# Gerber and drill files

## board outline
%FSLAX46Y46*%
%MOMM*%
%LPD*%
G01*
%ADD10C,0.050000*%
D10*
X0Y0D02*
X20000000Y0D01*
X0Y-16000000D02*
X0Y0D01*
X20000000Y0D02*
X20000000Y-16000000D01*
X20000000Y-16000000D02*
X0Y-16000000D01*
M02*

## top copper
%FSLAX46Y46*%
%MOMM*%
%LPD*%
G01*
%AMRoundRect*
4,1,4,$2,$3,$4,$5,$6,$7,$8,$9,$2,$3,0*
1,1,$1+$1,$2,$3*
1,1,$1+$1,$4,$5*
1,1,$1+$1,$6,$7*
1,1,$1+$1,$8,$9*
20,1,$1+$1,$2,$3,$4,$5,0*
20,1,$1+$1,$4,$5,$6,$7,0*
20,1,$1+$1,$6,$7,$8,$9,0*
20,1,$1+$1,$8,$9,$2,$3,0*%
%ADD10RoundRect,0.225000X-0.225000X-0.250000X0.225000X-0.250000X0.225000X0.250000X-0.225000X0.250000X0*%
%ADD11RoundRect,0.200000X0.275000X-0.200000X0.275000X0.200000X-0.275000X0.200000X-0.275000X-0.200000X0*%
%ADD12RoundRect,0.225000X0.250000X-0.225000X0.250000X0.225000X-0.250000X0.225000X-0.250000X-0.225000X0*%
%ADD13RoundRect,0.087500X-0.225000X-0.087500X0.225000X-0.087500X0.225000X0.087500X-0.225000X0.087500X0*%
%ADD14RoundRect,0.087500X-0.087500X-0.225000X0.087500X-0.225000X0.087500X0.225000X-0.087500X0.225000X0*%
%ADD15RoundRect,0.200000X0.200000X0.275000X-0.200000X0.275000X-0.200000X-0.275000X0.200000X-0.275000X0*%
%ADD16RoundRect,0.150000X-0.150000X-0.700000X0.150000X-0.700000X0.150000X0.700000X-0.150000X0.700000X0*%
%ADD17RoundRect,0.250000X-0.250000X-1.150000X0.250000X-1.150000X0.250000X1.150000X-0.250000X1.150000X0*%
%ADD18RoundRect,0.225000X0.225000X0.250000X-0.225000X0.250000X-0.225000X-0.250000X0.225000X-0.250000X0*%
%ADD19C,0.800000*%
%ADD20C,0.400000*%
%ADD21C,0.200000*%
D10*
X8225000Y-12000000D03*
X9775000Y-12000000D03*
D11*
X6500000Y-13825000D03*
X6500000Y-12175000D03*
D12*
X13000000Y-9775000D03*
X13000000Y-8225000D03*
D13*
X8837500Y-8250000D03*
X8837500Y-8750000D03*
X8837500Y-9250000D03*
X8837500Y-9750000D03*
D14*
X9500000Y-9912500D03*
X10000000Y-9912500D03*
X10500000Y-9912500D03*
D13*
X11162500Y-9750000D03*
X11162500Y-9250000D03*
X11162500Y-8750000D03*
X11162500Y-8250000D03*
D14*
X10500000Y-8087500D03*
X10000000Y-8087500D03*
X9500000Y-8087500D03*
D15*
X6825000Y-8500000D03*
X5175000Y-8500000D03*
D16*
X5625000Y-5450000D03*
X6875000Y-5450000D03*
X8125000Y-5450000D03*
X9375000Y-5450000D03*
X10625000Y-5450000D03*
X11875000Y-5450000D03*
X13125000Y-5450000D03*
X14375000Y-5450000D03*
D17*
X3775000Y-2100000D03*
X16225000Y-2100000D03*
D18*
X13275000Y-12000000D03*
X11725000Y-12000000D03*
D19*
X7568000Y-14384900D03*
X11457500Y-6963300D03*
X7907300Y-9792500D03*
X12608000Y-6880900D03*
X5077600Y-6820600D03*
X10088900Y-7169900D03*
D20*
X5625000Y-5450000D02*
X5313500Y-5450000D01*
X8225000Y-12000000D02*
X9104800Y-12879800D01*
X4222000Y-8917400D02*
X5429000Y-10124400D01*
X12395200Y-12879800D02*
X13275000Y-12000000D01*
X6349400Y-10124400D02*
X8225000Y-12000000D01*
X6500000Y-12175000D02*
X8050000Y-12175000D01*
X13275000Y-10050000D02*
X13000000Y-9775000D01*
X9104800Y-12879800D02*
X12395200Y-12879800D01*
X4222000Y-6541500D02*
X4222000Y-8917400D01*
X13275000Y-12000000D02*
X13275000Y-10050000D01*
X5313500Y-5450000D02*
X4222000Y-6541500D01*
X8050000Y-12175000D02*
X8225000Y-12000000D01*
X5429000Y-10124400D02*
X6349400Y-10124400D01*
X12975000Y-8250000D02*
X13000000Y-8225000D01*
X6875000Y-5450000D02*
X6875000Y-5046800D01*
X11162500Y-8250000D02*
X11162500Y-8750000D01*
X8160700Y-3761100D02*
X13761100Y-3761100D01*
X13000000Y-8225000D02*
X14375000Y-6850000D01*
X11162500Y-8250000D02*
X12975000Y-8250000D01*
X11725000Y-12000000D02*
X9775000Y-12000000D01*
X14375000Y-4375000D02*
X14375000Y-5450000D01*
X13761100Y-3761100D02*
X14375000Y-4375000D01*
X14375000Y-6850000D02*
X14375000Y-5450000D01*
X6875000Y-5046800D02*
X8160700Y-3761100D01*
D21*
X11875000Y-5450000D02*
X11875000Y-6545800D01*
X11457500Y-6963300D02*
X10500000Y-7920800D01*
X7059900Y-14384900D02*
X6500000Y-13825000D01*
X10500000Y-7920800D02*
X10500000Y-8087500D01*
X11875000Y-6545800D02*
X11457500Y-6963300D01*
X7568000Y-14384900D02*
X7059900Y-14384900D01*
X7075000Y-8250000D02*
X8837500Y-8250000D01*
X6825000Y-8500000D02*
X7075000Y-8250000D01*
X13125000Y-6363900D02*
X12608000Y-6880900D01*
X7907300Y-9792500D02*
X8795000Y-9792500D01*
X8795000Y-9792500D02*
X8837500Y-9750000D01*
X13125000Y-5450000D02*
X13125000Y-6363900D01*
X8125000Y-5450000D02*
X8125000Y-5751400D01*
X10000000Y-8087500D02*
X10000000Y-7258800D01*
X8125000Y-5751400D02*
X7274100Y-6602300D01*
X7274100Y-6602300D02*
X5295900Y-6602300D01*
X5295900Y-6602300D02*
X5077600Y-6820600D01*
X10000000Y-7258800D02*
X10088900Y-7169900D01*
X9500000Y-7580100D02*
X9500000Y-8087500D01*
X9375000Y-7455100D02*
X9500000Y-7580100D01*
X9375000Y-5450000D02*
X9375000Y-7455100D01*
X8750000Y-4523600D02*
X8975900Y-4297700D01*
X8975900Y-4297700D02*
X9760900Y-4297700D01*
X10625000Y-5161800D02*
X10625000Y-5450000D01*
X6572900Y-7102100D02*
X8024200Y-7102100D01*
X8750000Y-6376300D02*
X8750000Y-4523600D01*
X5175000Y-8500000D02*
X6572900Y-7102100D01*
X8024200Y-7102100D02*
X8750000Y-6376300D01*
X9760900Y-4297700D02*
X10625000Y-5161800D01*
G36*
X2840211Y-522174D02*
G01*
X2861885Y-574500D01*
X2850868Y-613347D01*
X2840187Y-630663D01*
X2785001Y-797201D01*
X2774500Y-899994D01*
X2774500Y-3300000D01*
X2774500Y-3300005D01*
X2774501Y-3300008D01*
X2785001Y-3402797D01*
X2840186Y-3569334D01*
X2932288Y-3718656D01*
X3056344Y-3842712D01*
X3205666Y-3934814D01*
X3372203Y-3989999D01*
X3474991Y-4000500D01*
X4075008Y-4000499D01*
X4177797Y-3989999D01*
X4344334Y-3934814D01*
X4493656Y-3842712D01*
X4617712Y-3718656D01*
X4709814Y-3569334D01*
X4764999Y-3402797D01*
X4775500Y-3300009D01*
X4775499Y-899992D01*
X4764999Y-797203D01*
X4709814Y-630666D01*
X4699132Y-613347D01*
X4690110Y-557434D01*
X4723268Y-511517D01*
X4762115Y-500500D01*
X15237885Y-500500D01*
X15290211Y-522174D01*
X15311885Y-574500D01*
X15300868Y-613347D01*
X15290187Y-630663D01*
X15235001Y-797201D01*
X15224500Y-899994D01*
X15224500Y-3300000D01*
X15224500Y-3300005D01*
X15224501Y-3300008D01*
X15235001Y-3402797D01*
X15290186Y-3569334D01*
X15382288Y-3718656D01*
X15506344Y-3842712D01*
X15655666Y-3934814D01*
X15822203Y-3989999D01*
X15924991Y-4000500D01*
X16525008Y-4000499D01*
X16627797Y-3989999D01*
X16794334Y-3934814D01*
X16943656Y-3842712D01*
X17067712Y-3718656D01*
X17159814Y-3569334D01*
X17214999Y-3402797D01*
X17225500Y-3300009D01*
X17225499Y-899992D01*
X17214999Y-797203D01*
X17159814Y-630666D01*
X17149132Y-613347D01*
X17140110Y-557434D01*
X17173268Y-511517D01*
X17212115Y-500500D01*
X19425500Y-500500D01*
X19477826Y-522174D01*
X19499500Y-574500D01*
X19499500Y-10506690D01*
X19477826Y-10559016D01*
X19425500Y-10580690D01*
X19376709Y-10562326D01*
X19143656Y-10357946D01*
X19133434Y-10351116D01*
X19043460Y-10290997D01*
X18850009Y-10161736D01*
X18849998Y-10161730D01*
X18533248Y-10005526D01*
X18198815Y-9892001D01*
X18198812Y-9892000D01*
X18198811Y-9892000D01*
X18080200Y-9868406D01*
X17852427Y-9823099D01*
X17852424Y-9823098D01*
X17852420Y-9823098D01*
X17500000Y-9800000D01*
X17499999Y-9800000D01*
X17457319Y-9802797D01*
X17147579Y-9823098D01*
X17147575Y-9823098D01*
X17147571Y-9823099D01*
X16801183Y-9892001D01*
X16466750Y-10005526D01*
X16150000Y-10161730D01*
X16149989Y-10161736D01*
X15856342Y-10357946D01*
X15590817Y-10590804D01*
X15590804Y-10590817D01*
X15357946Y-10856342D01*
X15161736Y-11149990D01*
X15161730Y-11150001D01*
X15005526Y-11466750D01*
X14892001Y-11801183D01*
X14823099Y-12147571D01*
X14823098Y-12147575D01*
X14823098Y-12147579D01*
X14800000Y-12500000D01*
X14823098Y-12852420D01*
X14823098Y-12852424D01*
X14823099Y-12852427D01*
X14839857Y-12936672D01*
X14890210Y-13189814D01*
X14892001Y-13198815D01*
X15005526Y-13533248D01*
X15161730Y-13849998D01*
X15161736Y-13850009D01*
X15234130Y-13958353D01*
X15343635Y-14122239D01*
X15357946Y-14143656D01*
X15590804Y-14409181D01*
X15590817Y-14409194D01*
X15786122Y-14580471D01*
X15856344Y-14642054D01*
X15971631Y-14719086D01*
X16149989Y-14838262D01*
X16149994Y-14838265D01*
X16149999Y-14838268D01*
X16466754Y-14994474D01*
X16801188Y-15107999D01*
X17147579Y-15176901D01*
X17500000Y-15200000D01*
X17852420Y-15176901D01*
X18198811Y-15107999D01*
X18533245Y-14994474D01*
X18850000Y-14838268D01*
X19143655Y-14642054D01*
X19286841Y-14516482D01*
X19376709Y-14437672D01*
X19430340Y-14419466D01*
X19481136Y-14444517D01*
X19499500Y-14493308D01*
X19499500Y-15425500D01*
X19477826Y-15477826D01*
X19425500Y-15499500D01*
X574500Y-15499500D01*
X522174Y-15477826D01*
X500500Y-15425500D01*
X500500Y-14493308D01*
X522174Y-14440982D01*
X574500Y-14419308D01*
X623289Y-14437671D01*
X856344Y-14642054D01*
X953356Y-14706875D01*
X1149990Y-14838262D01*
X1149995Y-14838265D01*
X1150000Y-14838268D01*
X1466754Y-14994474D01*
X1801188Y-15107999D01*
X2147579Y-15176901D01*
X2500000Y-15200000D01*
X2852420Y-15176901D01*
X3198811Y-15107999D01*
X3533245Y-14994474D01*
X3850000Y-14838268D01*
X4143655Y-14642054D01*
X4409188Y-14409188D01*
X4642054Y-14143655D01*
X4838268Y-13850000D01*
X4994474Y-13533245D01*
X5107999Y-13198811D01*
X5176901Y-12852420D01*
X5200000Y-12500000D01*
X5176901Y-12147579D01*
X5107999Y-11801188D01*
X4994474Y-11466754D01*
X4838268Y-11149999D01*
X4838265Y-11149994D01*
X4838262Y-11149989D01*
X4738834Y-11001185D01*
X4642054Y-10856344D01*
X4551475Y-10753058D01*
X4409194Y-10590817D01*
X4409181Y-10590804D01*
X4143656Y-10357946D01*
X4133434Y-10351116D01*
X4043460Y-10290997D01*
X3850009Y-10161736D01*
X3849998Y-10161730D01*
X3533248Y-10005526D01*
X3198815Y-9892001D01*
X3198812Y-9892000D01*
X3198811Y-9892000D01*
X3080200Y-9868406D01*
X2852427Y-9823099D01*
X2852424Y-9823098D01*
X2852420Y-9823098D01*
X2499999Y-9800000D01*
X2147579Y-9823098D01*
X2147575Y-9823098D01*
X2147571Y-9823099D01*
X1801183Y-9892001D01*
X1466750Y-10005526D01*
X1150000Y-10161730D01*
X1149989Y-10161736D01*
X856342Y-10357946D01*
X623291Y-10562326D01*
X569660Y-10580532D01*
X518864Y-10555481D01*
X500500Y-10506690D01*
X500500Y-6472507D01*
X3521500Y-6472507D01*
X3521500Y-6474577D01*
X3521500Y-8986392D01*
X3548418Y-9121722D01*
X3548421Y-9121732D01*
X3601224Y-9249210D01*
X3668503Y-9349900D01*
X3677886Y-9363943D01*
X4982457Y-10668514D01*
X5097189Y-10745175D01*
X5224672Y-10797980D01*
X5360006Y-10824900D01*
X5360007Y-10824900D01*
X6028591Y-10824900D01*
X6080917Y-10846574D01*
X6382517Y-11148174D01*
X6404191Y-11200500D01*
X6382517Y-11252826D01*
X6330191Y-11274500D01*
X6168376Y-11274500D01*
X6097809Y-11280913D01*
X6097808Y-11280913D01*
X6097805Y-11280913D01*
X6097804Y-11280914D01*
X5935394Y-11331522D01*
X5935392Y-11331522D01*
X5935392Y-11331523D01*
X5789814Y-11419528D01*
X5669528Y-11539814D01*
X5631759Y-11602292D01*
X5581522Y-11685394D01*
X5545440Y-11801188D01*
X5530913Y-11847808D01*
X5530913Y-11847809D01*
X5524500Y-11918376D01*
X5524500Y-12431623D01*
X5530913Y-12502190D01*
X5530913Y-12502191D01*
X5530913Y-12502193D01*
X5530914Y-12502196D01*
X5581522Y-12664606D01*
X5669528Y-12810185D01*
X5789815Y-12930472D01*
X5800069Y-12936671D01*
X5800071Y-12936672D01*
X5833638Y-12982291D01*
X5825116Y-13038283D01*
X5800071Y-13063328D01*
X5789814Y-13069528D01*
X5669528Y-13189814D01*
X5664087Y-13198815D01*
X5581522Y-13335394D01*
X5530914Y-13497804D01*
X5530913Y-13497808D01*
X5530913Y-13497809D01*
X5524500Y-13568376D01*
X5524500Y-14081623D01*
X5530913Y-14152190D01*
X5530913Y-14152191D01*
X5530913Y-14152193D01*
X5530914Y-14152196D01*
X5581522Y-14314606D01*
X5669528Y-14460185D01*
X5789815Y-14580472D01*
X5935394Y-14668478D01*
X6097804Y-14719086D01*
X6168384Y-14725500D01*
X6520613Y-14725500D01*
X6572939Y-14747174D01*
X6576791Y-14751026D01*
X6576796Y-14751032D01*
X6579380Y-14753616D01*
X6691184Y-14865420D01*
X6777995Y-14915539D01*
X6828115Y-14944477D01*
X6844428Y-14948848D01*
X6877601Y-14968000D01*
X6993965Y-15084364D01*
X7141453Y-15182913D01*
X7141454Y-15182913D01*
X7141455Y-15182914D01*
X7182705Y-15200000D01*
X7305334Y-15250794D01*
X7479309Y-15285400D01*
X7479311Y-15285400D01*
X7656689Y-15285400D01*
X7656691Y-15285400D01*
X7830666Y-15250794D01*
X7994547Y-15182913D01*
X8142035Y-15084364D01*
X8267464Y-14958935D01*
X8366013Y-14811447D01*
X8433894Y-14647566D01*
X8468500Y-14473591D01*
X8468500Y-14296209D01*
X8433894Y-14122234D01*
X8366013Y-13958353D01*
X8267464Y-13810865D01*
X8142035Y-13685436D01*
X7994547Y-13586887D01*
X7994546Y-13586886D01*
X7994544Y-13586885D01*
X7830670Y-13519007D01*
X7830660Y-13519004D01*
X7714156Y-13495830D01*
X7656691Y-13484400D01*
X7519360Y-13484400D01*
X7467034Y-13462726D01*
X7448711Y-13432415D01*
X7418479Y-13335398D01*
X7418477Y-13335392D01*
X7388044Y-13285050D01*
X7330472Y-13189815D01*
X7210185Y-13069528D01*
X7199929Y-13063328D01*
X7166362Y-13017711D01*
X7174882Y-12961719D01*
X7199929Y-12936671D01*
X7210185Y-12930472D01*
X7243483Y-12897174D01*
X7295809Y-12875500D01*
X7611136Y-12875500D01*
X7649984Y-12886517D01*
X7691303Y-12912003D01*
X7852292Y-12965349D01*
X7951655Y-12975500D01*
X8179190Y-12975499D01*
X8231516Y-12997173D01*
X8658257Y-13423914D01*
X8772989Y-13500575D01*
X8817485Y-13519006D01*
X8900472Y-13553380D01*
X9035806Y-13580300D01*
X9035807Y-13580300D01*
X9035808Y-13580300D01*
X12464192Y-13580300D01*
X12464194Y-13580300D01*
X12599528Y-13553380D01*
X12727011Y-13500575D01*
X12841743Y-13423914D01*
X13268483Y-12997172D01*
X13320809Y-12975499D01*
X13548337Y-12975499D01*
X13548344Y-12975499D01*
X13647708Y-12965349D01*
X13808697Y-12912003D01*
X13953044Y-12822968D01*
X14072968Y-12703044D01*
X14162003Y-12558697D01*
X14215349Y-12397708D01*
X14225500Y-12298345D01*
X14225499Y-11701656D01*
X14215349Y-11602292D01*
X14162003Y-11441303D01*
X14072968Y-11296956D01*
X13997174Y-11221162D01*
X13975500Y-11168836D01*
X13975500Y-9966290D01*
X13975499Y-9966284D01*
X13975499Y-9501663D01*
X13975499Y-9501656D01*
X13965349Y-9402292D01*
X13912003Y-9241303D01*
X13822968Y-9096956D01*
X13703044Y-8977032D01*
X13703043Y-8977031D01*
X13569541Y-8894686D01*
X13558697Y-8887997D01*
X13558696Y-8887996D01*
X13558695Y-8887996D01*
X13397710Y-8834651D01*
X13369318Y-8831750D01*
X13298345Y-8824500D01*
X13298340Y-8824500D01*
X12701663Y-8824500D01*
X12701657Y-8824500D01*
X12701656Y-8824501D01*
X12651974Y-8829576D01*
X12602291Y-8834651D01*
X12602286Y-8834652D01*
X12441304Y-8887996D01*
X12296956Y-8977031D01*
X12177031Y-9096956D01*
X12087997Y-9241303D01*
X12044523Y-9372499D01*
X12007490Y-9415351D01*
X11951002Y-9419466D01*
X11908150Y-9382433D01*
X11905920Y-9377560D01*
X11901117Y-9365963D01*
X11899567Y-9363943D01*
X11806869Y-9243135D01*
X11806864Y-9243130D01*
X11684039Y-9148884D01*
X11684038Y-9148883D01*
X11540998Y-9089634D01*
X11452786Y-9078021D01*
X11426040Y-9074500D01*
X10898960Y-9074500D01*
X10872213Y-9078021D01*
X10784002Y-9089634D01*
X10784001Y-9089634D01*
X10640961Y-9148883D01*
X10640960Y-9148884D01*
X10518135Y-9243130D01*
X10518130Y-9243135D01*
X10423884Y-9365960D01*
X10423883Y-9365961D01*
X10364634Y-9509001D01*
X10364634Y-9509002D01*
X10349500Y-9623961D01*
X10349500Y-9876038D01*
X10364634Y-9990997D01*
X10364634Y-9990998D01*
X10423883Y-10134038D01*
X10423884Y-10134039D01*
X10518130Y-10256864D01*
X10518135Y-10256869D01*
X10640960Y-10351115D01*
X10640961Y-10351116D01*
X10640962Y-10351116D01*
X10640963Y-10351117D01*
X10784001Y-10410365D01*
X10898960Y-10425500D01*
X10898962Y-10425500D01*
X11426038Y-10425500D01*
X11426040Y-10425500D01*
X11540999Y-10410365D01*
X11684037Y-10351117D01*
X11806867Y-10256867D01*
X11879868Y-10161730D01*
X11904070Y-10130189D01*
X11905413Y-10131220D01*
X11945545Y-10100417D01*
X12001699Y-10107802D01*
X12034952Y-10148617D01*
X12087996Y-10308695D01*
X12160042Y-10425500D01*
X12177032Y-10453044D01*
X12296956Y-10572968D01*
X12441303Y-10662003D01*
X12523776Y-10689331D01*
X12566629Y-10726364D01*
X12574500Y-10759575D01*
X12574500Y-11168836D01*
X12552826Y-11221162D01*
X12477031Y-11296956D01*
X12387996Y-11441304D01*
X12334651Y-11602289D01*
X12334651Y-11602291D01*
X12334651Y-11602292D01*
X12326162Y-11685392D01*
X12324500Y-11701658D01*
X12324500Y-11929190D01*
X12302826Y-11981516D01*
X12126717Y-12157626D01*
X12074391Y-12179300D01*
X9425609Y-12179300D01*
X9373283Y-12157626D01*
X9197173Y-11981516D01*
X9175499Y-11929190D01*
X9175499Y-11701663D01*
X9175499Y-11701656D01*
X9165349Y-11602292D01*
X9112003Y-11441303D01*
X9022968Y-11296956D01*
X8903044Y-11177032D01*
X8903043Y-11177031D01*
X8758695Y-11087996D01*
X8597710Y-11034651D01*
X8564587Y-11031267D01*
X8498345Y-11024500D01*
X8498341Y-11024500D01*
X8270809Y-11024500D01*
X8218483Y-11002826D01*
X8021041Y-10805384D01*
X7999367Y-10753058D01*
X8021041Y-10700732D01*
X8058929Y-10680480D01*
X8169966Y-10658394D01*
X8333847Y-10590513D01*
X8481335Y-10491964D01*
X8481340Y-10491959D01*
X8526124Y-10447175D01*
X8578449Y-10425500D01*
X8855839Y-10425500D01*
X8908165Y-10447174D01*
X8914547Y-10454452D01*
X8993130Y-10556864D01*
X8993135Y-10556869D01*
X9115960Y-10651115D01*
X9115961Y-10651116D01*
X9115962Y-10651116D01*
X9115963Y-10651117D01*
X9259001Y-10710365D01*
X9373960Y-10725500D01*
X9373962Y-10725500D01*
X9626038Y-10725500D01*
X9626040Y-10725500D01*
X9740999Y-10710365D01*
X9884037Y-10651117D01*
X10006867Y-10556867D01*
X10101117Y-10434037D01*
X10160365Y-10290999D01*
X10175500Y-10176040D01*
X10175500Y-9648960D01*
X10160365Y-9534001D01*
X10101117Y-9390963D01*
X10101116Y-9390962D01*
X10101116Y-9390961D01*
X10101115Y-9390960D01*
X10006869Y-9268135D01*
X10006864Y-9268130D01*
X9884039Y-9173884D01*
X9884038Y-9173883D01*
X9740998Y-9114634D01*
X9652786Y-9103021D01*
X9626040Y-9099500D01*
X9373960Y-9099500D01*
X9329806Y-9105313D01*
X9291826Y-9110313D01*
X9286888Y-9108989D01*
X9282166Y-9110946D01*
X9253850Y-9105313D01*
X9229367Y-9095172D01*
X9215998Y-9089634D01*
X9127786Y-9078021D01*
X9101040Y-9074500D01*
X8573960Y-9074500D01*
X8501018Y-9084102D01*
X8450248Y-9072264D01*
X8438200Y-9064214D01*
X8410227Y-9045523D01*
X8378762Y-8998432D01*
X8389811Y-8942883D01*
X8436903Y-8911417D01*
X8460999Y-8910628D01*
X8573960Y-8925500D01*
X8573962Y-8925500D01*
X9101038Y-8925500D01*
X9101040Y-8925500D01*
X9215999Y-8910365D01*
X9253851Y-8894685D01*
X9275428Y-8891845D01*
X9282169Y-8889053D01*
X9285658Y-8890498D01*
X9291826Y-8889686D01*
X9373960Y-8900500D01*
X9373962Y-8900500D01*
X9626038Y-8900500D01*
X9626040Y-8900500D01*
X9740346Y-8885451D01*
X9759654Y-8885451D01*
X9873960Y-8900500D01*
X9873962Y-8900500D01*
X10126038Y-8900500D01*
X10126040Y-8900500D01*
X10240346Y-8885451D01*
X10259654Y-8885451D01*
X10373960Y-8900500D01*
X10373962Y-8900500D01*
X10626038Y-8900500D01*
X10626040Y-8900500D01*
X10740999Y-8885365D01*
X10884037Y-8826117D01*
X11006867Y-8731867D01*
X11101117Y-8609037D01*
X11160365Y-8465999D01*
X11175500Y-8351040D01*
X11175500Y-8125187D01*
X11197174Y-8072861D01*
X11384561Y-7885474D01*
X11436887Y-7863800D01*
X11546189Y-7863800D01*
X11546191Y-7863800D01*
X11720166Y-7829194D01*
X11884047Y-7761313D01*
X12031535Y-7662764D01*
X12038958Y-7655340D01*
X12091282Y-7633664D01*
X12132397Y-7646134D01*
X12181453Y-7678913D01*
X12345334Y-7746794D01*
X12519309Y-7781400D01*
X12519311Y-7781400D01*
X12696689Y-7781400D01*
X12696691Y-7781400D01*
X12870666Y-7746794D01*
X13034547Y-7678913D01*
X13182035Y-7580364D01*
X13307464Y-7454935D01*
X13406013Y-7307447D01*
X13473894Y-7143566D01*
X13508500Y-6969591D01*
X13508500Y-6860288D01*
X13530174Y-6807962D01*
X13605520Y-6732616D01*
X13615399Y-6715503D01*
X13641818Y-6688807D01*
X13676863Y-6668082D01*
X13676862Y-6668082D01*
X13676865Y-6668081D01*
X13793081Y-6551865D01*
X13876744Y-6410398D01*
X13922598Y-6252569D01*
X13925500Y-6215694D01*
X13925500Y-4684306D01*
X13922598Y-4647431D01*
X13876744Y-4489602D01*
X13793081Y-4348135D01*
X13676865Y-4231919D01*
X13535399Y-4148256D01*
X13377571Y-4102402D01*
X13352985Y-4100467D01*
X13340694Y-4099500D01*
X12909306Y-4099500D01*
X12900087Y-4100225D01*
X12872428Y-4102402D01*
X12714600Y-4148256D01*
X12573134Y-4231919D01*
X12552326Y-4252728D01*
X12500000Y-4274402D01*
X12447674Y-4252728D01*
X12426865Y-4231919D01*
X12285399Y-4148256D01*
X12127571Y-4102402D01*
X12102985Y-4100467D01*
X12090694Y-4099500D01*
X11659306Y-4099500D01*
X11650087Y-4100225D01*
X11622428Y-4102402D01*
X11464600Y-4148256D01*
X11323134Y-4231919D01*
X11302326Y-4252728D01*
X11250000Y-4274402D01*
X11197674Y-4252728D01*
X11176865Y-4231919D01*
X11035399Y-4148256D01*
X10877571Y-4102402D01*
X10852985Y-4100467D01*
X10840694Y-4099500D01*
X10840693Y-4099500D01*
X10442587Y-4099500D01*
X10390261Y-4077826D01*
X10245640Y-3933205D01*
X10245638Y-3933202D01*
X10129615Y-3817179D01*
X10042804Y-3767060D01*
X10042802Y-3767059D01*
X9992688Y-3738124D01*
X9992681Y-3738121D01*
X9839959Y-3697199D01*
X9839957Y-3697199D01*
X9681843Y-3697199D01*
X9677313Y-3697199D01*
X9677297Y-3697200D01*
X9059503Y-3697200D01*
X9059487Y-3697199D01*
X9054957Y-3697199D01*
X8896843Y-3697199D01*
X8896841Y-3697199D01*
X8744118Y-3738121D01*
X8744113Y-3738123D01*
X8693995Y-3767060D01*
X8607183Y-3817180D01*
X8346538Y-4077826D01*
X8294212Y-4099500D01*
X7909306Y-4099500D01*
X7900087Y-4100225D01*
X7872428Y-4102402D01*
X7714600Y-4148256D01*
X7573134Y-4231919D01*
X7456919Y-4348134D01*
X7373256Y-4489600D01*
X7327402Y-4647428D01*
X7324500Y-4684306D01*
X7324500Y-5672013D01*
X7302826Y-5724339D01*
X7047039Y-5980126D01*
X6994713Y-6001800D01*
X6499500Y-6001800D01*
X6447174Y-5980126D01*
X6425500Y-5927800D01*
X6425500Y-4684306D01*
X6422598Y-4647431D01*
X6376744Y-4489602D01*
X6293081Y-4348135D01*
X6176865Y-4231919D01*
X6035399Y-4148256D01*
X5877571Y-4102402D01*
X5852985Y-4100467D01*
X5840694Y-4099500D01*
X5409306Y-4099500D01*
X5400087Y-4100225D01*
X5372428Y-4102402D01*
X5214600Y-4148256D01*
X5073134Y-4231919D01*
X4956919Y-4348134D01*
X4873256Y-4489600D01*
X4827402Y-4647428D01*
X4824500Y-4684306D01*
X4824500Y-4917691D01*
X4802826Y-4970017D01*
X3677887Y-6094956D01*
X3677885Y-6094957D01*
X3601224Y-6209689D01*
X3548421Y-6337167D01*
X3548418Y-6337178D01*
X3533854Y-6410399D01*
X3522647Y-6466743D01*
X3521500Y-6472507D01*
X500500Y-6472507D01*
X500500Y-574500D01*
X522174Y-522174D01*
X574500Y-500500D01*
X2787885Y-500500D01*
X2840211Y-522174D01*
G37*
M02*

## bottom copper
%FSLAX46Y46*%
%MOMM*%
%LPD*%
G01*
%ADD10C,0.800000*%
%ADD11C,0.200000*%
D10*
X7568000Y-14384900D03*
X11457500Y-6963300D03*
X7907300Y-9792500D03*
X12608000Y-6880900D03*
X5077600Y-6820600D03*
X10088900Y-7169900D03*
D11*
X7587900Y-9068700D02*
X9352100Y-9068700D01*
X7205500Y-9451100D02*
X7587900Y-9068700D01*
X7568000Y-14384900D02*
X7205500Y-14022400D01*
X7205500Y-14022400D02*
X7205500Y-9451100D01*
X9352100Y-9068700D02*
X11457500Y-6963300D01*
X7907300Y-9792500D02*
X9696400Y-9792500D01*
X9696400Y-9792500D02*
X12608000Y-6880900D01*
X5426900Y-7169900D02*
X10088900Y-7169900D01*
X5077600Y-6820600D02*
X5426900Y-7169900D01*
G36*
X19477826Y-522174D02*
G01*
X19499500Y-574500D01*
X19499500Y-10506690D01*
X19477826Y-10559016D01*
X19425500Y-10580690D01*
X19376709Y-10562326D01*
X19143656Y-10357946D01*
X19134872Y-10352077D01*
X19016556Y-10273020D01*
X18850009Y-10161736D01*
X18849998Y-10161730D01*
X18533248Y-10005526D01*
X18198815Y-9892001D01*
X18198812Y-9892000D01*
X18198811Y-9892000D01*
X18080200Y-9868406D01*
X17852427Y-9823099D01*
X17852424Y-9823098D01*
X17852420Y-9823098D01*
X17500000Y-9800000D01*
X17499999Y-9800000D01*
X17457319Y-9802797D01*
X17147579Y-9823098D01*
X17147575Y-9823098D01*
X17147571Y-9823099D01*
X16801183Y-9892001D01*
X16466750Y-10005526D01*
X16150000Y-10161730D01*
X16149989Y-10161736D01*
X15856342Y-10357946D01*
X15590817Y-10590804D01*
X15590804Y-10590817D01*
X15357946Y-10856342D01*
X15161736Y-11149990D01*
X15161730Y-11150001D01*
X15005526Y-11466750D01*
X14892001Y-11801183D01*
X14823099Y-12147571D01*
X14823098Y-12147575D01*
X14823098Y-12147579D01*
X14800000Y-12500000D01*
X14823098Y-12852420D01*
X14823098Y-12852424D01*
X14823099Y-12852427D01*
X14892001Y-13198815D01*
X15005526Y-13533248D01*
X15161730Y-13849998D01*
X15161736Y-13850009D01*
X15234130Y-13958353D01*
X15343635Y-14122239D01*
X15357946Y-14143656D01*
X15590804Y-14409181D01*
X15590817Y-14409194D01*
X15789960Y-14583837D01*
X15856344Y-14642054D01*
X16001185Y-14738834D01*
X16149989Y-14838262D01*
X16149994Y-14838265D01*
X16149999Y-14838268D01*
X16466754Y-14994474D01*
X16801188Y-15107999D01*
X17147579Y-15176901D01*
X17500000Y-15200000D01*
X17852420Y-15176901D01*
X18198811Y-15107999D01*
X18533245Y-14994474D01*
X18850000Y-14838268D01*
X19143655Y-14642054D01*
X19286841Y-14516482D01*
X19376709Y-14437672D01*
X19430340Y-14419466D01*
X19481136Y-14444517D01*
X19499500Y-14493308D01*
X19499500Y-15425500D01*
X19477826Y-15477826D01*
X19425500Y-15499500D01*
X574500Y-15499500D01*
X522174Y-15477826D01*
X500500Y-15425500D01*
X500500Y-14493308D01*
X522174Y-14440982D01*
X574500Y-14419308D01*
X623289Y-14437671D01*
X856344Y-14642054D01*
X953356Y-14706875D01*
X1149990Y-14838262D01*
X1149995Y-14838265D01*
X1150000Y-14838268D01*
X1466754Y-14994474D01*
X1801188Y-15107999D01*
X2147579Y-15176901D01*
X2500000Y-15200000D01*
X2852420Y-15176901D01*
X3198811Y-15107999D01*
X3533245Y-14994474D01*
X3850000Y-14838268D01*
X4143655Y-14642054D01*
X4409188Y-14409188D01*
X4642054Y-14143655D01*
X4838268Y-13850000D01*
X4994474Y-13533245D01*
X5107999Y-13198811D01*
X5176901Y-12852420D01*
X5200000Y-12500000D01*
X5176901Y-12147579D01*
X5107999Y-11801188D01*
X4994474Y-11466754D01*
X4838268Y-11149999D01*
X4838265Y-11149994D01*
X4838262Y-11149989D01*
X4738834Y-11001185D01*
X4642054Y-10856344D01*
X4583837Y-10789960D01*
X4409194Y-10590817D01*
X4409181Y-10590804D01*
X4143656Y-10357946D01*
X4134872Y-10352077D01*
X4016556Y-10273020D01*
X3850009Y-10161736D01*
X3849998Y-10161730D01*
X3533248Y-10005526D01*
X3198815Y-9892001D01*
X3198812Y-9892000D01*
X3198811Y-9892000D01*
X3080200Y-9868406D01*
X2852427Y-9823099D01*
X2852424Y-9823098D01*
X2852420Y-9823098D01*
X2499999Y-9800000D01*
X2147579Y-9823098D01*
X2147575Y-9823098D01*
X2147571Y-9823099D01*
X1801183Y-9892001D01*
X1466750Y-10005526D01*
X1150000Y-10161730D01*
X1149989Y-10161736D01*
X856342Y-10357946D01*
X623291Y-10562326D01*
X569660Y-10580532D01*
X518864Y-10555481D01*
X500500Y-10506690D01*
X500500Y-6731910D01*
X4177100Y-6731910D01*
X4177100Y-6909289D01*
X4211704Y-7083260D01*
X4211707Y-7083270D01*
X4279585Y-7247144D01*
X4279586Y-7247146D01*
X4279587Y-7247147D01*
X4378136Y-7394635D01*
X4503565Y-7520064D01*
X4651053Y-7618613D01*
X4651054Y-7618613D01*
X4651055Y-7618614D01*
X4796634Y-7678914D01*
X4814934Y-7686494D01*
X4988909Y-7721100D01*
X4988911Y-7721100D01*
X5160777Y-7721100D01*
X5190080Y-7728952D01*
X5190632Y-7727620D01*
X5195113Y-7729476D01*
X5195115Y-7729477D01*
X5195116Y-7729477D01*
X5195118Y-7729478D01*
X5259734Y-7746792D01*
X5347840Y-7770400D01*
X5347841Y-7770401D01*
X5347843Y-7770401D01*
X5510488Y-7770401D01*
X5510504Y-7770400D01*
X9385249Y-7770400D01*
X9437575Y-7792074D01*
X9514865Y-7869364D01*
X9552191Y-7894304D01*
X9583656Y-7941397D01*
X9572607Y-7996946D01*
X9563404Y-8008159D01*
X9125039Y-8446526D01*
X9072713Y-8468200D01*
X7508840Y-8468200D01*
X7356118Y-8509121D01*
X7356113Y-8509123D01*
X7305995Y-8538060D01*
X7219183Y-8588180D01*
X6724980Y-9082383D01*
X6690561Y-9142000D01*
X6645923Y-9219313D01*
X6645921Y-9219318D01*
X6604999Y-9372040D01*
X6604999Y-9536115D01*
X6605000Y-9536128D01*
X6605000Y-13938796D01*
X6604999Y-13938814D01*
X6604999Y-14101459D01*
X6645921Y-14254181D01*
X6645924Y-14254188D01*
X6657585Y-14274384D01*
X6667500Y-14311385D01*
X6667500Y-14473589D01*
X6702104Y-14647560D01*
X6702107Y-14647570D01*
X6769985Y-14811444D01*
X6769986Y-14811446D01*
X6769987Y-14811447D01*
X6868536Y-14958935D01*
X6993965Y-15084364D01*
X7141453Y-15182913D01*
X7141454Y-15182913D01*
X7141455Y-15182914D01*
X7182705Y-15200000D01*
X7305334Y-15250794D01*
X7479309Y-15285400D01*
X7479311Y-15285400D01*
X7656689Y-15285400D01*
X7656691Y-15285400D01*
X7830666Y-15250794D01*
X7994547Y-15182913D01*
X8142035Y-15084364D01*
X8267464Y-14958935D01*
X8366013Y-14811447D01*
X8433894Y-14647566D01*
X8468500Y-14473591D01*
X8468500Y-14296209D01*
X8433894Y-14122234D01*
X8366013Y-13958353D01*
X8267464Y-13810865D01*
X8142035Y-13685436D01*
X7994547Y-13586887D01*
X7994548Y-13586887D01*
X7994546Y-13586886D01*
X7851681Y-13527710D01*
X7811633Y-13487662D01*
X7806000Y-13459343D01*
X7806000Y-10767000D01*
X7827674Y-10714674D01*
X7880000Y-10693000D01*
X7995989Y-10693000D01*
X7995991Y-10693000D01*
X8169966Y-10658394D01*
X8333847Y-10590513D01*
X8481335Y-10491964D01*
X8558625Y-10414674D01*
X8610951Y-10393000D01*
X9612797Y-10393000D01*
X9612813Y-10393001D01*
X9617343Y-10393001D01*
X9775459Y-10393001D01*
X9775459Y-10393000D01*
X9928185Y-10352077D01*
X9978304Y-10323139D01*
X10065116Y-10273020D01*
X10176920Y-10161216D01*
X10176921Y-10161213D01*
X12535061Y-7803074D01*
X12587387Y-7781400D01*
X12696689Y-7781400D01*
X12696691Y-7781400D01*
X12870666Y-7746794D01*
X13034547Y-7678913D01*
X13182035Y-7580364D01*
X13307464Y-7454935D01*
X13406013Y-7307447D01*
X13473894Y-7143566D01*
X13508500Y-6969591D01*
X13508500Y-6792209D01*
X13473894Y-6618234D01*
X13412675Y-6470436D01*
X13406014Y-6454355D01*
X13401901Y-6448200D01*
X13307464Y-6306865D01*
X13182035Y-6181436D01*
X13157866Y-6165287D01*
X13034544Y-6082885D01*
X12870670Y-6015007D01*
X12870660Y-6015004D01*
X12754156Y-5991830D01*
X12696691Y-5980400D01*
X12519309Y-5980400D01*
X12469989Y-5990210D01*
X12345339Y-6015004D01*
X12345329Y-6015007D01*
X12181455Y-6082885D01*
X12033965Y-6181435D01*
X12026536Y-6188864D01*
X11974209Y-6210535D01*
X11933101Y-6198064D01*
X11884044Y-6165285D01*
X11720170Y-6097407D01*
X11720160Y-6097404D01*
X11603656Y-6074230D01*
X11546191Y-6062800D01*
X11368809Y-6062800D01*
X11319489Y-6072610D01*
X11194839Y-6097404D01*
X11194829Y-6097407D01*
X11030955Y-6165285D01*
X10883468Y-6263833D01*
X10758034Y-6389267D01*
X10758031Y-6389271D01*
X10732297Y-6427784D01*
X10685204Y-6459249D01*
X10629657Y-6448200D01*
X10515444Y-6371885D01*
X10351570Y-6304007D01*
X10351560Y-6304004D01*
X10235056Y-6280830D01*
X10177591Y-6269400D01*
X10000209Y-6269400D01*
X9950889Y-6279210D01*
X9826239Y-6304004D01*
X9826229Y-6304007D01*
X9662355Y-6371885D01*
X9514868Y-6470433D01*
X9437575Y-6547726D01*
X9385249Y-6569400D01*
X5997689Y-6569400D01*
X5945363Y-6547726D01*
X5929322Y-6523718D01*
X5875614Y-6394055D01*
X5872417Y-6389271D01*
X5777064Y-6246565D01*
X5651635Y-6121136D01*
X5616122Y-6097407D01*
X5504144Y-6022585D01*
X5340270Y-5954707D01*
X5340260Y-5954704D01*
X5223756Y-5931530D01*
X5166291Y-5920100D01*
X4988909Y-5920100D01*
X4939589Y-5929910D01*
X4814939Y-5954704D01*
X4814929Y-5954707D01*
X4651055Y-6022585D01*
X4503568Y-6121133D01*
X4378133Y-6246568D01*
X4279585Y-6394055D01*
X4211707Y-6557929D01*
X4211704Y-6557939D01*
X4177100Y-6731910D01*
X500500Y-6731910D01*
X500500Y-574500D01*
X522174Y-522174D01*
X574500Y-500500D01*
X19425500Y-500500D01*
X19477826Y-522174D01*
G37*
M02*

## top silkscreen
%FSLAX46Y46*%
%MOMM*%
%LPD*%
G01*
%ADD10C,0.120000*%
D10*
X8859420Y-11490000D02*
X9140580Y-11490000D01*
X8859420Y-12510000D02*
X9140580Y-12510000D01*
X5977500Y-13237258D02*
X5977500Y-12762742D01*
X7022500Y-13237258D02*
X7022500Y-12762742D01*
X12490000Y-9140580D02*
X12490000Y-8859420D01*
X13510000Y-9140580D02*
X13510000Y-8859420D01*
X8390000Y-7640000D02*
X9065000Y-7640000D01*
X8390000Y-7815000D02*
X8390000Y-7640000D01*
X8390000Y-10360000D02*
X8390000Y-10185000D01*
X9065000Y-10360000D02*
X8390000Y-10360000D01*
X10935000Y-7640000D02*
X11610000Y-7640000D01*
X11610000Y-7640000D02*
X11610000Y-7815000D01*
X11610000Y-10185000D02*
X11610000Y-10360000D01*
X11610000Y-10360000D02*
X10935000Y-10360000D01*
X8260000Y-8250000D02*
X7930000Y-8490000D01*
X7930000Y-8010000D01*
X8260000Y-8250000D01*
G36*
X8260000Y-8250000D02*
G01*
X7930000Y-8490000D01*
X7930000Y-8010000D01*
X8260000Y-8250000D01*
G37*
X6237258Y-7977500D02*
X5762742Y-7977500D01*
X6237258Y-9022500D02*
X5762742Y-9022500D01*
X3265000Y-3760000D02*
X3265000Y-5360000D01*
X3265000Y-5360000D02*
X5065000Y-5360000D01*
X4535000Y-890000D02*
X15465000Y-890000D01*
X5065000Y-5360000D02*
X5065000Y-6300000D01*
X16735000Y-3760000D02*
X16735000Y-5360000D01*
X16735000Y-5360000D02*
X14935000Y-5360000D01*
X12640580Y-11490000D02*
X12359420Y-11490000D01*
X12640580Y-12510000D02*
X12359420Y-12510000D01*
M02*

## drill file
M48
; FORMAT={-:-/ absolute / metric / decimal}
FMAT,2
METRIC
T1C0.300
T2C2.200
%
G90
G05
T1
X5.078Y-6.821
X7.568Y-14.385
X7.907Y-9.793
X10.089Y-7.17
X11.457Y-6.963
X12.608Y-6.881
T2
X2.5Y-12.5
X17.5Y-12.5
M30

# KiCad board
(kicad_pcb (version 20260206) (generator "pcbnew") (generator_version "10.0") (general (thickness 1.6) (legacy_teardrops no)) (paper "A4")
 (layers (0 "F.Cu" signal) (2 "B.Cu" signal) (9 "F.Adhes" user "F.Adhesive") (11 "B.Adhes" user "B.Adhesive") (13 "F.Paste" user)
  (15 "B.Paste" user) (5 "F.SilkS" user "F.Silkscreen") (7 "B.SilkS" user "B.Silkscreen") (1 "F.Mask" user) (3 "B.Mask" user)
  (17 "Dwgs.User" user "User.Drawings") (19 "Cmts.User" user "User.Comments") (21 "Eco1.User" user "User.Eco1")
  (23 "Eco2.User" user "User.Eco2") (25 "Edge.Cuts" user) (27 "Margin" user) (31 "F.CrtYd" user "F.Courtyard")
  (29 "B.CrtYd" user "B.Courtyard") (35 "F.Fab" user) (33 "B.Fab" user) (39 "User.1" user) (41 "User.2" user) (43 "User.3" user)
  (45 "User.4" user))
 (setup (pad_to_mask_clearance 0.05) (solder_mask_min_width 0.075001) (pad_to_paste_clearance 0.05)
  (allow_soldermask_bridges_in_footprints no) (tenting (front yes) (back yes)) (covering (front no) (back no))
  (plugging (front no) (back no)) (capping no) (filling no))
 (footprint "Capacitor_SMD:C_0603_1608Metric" (layer "F.Cu") (at 9 12)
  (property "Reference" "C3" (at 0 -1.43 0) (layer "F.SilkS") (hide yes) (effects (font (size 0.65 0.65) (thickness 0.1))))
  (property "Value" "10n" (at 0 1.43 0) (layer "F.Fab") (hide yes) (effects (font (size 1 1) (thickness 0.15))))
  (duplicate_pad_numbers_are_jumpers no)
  (fp_line (start -0.14058 -0.51) (end 0.14058 -0.51) (stroke (width 0.12) (type solid)) (layer "F.SilkS"))
  (fp_line (start -0.14058 0.51) (end 0.14058 0.51) (stroke (width 0.12) (type solid)) (layer "F.SilkS"))
  (pad "1" smd roundrect (at -0.775 0) (size 0.9 0.95) (layers "F.Cu" "F.Mask" "F.Paste") (roundrect_rratio 0.25) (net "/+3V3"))
  (pad "2" smd roundrect (at 0.775 0) (size 0.9 0.95) (layers "F.Cu" "F.Mask" "F.Paste") (roundrect_rratio 0.25) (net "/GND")
   (zone_connect 2)))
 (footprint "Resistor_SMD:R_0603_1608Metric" (layer "F.Cu") (at 6.5 13 90)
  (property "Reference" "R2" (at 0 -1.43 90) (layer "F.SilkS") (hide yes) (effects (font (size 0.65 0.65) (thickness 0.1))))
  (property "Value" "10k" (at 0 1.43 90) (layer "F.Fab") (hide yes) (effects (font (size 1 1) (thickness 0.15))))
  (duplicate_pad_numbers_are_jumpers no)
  (fp_line (start -0.237258 -0.5225) (end 0.237258 -0.5225) (stroke (width 0.12) (type solid)) (layer "F.SilkS"))
  (fp_line (start -0.237258 0.5225) (end 0.237258 0.5225) (stroke (width 0.12) (type solid)) (layer "F.SilkS"))
  (pad "1" smd roundrect (at -0.825 0 90) (size 0.8 0.95) (layers "F.Cu" "F.Mask" "F.Paste") (roundrect_rratio 0.25) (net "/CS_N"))
  (pad "2" smd roundrect (at 0.825 0 90) (size 0.8 0.95) (layers "F.Cu" "F.Mask" "F.Paste") (roundrect_rratio 0.25) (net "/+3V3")))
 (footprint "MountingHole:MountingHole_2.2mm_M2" (layer "F.Cu") (at 2.5 12.5)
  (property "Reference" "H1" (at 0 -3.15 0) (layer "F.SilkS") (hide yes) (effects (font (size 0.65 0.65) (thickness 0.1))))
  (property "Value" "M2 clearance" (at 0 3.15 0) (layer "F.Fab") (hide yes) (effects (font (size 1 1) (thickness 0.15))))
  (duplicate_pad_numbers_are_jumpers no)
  (pad "" np_thru_hole circle (at 0 0) (size 2.2 2.2) (drill 2.2) (layers "*.Cu" "*.Mask")))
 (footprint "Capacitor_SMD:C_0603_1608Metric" (layer "F.Cu") (at 13 9 90)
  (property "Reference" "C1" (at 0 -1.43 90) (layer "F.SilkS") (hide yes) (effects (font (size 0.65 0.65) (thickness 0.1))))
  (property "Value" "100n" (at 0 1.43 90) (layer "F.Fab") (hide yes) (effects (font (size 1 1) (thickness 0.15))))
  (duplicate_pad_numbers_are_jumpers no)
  (fp_line (start -0.14058 -0.51) (end 0.14058 -0.51) (stroke (width 0.12) (type solid)) (layer "F.SilkS"))
  (fp_line (start -0.14058 0.51) (end 0.14058 0.51) (stroke (width 0.12) (type solid)) (layer "F.SilkS"))
  (pad "1" smd roundrect (at -0.775 0 90) (size 0.9 0.95) (layers "F.Cu" "F.Mask" "F.Paste") (roundrect_rratio 0.25) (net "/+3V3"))
  (pad "2" smd roundrect (at 0.775 0 90) (size 0.9 0.95) (layers "F.Cu" "F.Mask" "F.Paste") (roundrect_rratio 0.25) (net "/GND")
   (zone_connect 2)))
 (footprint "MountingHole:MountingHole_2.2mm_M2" (layer "F.Cu") (at 17.5 12.5)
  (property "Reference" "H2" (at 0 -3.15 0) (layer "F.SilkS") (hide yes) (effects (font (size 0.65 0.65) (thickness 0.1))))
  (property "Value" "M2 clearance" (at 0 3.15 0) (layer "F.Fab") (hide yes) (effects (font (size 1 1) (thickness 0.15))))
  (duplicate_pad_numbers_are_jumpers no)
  (pad "" np_thru_hole circle (at 0 0) (size 2.2 2.2) (drill 2.2) (layers "*.Cu" "*.Mask")))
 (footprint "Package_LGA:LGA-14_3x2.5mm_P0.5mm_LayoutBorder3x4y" (layer "F.Cu") (at 10 9)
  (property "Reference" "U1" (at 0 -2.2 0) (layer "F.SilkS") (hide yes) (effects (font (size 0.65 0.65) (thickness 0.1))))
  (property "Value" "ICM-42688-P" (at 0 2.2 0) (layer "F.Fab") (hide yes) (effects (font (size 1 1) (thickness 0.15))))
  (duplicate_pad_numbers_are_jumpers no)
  (fp_line (start -1.61 -1.36) (end -0.935 -1.36) (stroke (width 0.12) (type solid)) (layer "F.SilkS"))
  (fp_line (start -1.61 -1.185) (end -1.61 -1.36) (stroke (width 0.12) (type solid)) (layer "F.SilkS"))
  (fp_line (start -1.61 1.36) (end -1.61 1.185) (stroke (width 0.12) (type solid)) (layer "F.SilkS"))
  (fp_line (start -0.935 1.36) (end -1.61 1.36) (stroke (width 0.12) (type solid)) (layer "F.SilkS"))
  (fp_line (start 0.935 -1.36) (end 1.61 -1.36) (stroke (width 0.12) (type solid)) (layer "F.SilkS"))
  (fp_line (start 1.61 -1.36) (end 1.61 -1.185) (stroke (width 0.12) (type solid)) (layer "F.SilkS"))
  (fp_line (start 1.61 1.185) (end 1.61 1.36) (stroke (width 0.12) (type solid)) (layer "F.SilkS"))
  (fp_line (start 1.61 1.36) (end 0.935 1.36) (stroke (width 0.12) (type solid)) (layer "F.SilkS"))
  (fp_poly (pts (xy -1.74 -0.75) (xy -2.07 -0.51) (xy -2.07 -0.99)) (stroke (width 0.12) (type solid)) (fill yes) (layer "F.SilkS"))
  (pad "1" smd roundrect (at -1.1625 -0.75) (size 0.625 0.35) (layers "F.Cu" "F.Mask" "F.Paste") (roundrect_rratio 0.25) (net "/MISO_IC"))
  (pad "2" smd roundrect (at -1.1625 -0.25) (size 0.625 0.35) (layers "F.Cu" "F.Mask" "F.Paste") (roundrect_rratio 0.25) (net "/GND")
   (zone_connect 2))
  (pad "3" smd roundrect (at -1.1625 0.25) (size 0.625 0.35) (layers "F.Cu" "F.Mask" "F.Paste") (roundrect_rratio 0.25) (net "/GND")
   (zone_connect 2))
  (pad "4" smd roundrect (at -1.1625 0.75) (size 0.625 0.35) (layers "F.Cu" "F.Mask" "F.Paste") (roundrect_rratio 0.25) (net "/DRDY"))
  (pad "5" smd roundrect (at -0.5 0.9125) (size 0.35 0.625) (layers "F.Cu" "F.Mask" "F.Paste") (roundrect_rratio 0.25) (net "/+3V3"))
  (pad "6" smd roundrect (at 0 0.9125) (size 0.35 0.625) (layers "F.Cu" "F.Mask" "F.Paste") (roundrect_rratio 0.25) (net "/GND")
   (zone_connect 2))
  (pad "7" smd roundrect (at 0.5 0.9125) (size 0.35 0.625) (layers "F.Cu" "F.Mask" "F.Paste") (roundrect_rratio 0.25) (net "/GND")
   (zone_connect 2))
  (pad "8" smd roundrect (at 1.1625 0.75) (size 0.625 0.35) (layers "F.Cu" "F.Mask" "F.Paste") (roundrect_rratio 0.25) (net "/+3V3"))
  (pad "9" smd roundrect (at 1.1625 0.25) (size 0.625 0.35) (layers "F.Cu" "F.Mask" "F.Paste") (roundrect_rratio 0.25) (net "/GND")
   (zone_connect 2))
  (pad "10" smd roundrect (at 1.1625 -0.25) (size 0.625 0.35) (layers "F.Cu" "F.Mask" "F.Paste") (roundrect_rratio 0.25) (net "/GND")
   (zone_connect 2))
  (pad "11" smd roundrect (at 1.1625 -0.75) (size 0.625 0.35) (layers "F.Cu" "F.Mask" "F.Paste") (roundrect_rratio 0.25) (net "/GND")
   (zone_connect 2))
  (pad "12" smd roundrect (at 0.5 -0.9125) (size 0.35 0.625) (layers "F.Cu" "F.Mask" "F.Paste") (roundrect_rratio 0.25) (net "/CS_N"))
  (pad "13" smd roundrect (at 0 -0.9125) (size 0.35 0.625) (layers "F.Cu" "F.Mask" "F.Paste") (roundrect_rratio 0.25) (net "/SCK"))
  (pad "14" smd roundrect (at -0.5 -0.9125) (size 0.35 0.625) (layers "F.Cu" "F.Mask" "F.Paste") (roundrect_rratio 0.25) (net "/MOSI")))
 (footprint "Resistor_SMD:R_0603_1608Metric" (layer "F.Cu") (at 6 8.5 180)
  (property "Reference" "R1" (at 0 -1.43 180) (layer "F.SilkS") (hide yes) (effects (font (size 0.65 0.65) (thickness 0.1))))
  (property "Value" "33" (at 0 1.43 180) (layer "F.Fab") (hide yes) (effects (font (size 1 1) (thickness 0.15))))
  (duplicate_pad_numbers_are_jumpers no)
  (fp_line (start -0.237258 0.5225) (end 0.237258 0.5225) (stroke (width 0.12) (type solid)) (layer "F.SilkS"))
  (fp_line (start -0.237258 -0.5225) (end 0.237258 -0.5225) (stroke (width 0.12) (type solid)) (layer "F.SilkS"))
  (pad "1" smd roundrect (at -0.825 0 180) (size 0.8 0.95) (layers "F.Cu" "F.Mask" "F.Paste") (roundrect_rratio 0.25) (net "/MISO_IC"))
  (pad "2" smd roundrect (at 0.825 0 180) (size 0.8 0.95) (layers "F.Cu" "F.Mask" "F.Paste") (roundrect_rratio 0.25) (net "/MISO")))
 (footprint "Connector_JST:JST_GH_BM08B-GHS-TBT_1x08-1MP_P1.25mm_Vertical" (layer "F.Cu") (at 10 3.5)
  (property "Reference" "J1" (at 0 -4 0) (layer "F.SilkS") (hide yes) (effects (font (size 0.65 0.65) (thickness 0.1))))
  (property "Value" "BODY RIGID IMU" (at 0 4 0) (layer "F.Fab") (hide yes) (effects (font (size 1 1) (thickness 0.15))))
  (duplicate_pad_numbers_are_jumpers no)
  (fp_line (start -6.735 0.26) (end -6.735 1.86) (stroke (width 0.12) (type solid)) (layer "F.SilkS"))
  (fp_line (start -6.735 1.86) (end -4.935 1.86) (stroke (width 0.12) (type solid)) (layer "F.SilkS"))
  (fp_line (start -5.465 -2.61) (end 5.465 -2.61) (stroke (width 0.12) (type solid)) (layer "F.SilkS"))
  (fp_line (start -4.935 1.86) (end -4.935 2.8) (stroke (width 0.12) (type solid)) (layer "F.SilkS"))
  (fp_line (start 6.735 0.26) (end 6.735 1.86) (stroke (width 0.12) (type solid)) (layer "F.SilkS"))
  (fp_line (start 6.735 1.86) (end 4.935 1.86) (stroke (width 0.12) (type solid)) (layer "F.SilkS"))
  (pad "1" smd roundrect (at -4.375 1.95) (size 0.6 1.7) (layers "F.Cu" "F.Mask" "F.Paste") (roundrect_rratio 0.25) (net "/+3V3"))
  (pad "2" smd roundrect (at -3.125 1.95) (size 0.6 1.7) (layers "F.Cu" "F.Mask" "F.Paste") (roundrect_rratio 0.25) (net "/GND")
   (zone_connect 2))
  (pad "3" smd roundrect (at -1.875 1.95) (size 0.6 1.7) (layers "F.Cu" "F.Mask" "F.Paste") (roundrect_rratio 0.25) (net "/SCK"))
  (pad "4" smd roundrect (at -0.625 1.95) (size 0.6 1.7) (layers "F.Cu" "F.Mask" "F.Paste") (roundrect_rratio 0.25) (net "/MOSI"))
  (pad "5" smd roundrect (at 0.625 1.95) (size 0.6 1.7) (layers "F.Cu" "F.Mask" "F.Paste") (roundrect_rratio 0.25) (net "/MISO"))
  (pad "6" smd roundrect (at 1.875 1.95) (size 0.6 1.7) (layers "F.Cu" "F.Mask" "F.Paste") (roundrect_rratio 0.25) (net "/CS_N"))
  (pad "7" smd roundrect (at 3.125 1.95) (size 0.6 1.7) (layers "F.Cu" "F.Mask" "F.Paste") (roundrect_rratio 0.25) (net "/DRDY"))
  (pad "8" smd roundrect (at 4.375 1.95) (size 0.6 1.7) (layers "F.Cu" "F.Mask" "F.Paste") (roundrect_rratio 0.25) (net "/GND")
   (zone_connect 2))
  (pad "MP" smd roundrect (at -6.225 -1.4) (size 1 2.8) (layers "F.Cu" "F.Mask" "F.Paste") (roundrect_rratio 0.25))
  (pad "MP" smd roundrect (at 6.225 -1.4) (size 1 2.8) (layers "F.Cu" "F.Mask" "F.Paste") (roundrect_rratio 0.25)))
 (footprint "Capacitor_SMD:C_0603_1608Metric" (layer "F.Cu") (at 12.5 12 180)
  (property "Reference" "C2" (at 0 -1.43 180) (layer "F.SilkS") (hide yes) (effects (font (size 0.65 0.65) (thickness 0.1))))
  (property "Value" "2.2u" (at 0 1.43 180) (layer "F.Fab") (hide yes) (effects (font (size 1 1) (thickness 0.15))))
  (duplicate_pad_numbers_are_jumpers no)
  (fp_line (start -0.14058 0.51) (end 0.14058 0.51) (stroke (width 0.12) (type solid)) (layer "F.SilkS"))
  (fp_line (start -0.14058 -0.51) (end 0.14058 -0.51) (stroke (width 0.12) (type solid)) (layer "F.SilkS"))
  (pad "1" smd roundrect (at -0.775 0 180) (size 0.9 0.95) (layers "F.Cu" "F.Mask" "F.Paste") (roundrect_rratio 0.25) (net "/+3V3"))
  (pad "2" smd roundrect (at 0.775 0 180) (size 0.9 0.95) (layers "F.Cu" "F.Mask" "F.Paste") (roundrect_rratio 0.25) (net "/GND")
   (zone_connect 2)))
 (gr_line (start 0 0) (end 20 0) (stroke (width 0.05) (type default)) (layer "Edge.Cuts"))
 (gr_line (start 0 16) (end 0 0) (stroke (width 0.05) (type default)) (layer "Edge.Cuts"))
 (gr_line (start 20 0) (end 20 16) (stroke (width 0.05) (type default)) (layer "Edge.Cuts"))
 (gr_line (start 20 16) (end 0 16) (stroke (width 0.05) (type default)) (layer "Edge.Cuts"))
 (segment (start 5.625 5.45) (end 5.3135 5.45) (width 0.4) (layer "F.Cu") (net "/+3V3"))
 (segment (start 8.225 12) (end 9.1048 12.8798) (width 0.4) (layer "F.Cu") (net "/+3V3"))
 (segment (start 4.222 8.9174) (end 5.429 10.1244) (width 0.4) (layer "F.Cu") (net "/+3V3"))
 (segment (start 12.3952 12.8798) (end 13.275 12) (width 0.4) (layer "F.Cu") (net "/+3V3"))
 (segment (start 6.3494 10.1244) (end 8.225 12) (width 0.4) (layer "F.Cu") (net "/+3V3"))
 (segment (start 6.5 12.175) (end 8.05 12.175) (width 0.4) (layer "F.Cu") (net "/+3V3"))
 (segment (start 13.275 10.05) (end 13 9.775) (width 0.4) (layer "F.Cu") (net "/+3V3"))
 (segment (start 9.1048 12.8798) (end 12.3952 12.8798) (width 0.4) (layer "F.Cu") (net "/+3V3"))
 (segment (start 4.222 6.5415) (end 4.222 8.9174) (width 0.4) (layer "F.Cu") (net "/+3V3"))
 (segment (start 13.275 12) (end 13.275 10.05) (width 0.4) (layer "F.Cu") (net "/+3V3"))
 (segment (start 5.3135 5.45) (end 4.222 6.5415) (width 0.4) (layer "F.Cu") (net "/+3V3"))
 (segment (start 8.05 12.175) (end 8.225 12) (width 0.4) (layer "F.Cu") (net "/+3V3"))
 (segment (start 5.429 10.1244) (end 6.3494 10.1244) (width 0.4) (layer "F.Cu") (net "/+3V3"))
 (segment (start 12.975 8.25) (end 13 8.225) (width 0.4) (layer "F.Cu") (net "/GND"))
 (segment (start 6.875 5.45) (end 6.875 5.0468) (width 0.4) (layer "F.Cu") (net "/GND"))
 (segment (start 11.1625 8.25) (end 11.1625 8.75) (width 0.4) (layer "F.Cu") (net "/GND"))
 (segment (start 8.1607 3.7611) (end 13.7611 3.7611) (width 0.4) (layer "F.Cu") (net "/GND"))
 (segment (start 13 8.225) (end 14.375 6.85) (width 0.4) (layer "F.Cu") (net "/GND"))
 (segment (start 11.1625 8.25) (end 12.975 8.25) (width 0.4) (layer "F.Cu") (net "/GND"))
 (segment (start 11.725 12) (end 9.775 12) (width 0.4) (layer "F.Cu") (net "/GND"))
 (segment (start 14.375 4.375) (end 14.375 5.45) (width 0.4) (layer "F.Cu") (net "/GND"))
 (segment (start 13.7611 3.7611) (end 14.375 4.375) (width 0.4) (layer "F.Cu") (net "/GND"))
 (segment (start 14.375 6.85) (end 14.375 5.45) (width 0.4) (layer "F.Cu") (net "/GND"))
 (segment (start 6.875 5.0468) (end 8.1607 3.7611) (width 0.4) (layer "F.Cu") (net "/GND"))
 (segment (start 11.875 5.45) (end 11.875 6.5458) (width 0.2) (layer "F.Cu") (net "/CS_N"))
 (segment (start 11.4575 6.9633) (end 10.5 7.9208) (width 0.2) (layer "F.Cu") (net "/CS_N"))
 (segment (start 7.0599 14.3849) (end 6.5 13.825) (width 0.2) (layer "F.Cu") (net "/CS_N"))
 (segment (start 10.5 7.9208) (end 10.5 8.0875) (width 0.2) (layer "F.Cu") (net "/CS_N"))
 (segment (start 11.875 6.5458) (end 11.4575 6.9633) (width 0.2) (layer "F.Cu") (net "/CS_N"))
 (segment (start 7.568 14.3849) (end 7.0599 14.3849) (width 0.2) (layer "F.Cu") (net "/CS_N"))
 (via (at 7.568 14.3849) (size 0.8) (drill 0.3) (layers "F.Cu" "B.Cu") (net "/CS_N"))
 (via (at 11.4575 6.9633) (size 0.8) (drill 0.3) (layers "F.Cu" "B.Cu") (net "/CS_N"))
 (segment (start 7.5879 9.0687) (end 9.3521 9.0687) (width 0.2) (layer "B.Cu") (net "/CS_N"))
 (segment (start 7.2055 9.4511) (end 7.5879 9.0687) (width 0.2) (layer "B.Cu") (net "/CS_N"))
 (segment (start 7.568 14.3849) (end 7.2055 14.0224) (width 0.2) (layer "B.Cu") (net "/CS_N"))
 (segment (start 7.2055 14.0224) (end 7.2055 9.4511) (width 0.2) (layer "B.Cu") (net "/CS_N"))
 (segment (start 9.3521 9.0687) (end 11.4575 6.9633) (width 0.2) (layer "B.Cu") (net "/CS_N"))
 (segment (start 7.075 8.25) (end 8.8375 8.25) (width 0.2) (layer "F.Cu") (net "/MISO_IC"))
 (segment (start 6.825 8.5) (end 7.075 8.25) (width 0.2) (layer "F.Cu") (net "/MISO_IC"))
 (segment (start 13.125 6.3639) (end 12.608 6.8809) (width 0.2) (layer "F.Cu") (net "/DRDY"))
 (segment (start 7.9073 9.7925) (end 8.795 9.7925) (width 0.2) (layer "F.Cu") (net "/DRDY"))
 (segment (start 8.795 9.7925) (end 8.8375 9.75) (width 0.2) (layer "F.Cu") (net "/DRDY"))
 (segment (start 13.125 5.45) (end 13.125 6.3639) (width 0.2) (layer "F.Cu") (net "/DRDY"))
 (via (at 7.9073 9.7925) (size 0.8) (drill 0.3) (layers "F.Cu" "B.Cu") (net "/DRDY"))
 (via (at 12.608 6.8809) (size 0.8) (drill 0.3) (layers "F.Cu" "B.Cu") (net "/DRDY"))
 (segment (start 7.9073 9.7925) (end 9.6964 9.7925) (width 0.2) (layer "B.Cu") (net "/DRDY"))
 (segment (start 9.6964 9.7925) (end 12.608 6.8809) (width 0.2) (layer "B.Cu") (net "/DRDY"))
 (segment (start 8.125 5.45) (end 8.125 5.7514) (width 0.2) (layer "F.Cu") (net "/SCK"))
 (segment (start 10 8.0875) (end 10 7.2588) (width 0.2) (layer "F.Cu") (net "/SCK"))
 (segment (start 8.125 5.7514) (end 7.2741 6.6023) (width 0.2) (layer "F.Cu") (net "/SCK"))
 (segment (start 7.2741 6.6023) (end 5.2959 6.6023) (width 0.2) (layer "F.Cu") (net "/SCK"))
 (segment (start 5.2959 6.6023) (end 5.0776 6.8206) (width 0.2) (layer "F.Cu") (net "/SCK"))
 (segment (start 10 7.2588) (end 10.0889 7.1699) (width 0.2) (layer "F.Cu") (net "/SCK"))
 (via (at 5.0776 6.8206) (size 0.8) (drill 0.3) (layers "F.Cu" "B.Cu") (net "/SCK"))
 (via (at 10.0889 7.1699) (size 0.8) (drill 0.3) (layers "F.Cu" "B.Cu") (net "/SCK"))
 (segment (start 5.4269 7.1699) (end 10.0889 7.1699) (width 0.2) (layer "B.Cu") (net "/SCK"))
 (segment (start 5.0776 6.8206) (end 5.4269 7.1699) (width 0.2) (layer "B.Cu") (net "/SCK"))
 (segment (start 9.5 7.5801) (end 9.5 8.0875) (width 0.2) (layer "F.Cu") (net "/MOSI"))
 (segment (start 9.375 7.4551) (end 9.5 7.5801) (width 0.2) (layer "F.Cu") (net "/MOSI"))
 (segment (start 9.375 5.45) (end 9.375 7.4551) (width 0.2) (layer "F.Cu") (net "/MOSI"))
 (segment (start 8.75 4.5236) (end 8.9759 4.2977) (width 0.2) (layer "F.Cu") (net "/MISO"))
 (segment (start 8.9759 4.2977) (end 9.7609 4.2977) (width 0.2) (layer "F.Cu") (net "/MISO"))
 (segment (start 10.625 5.1618) (end 10.625 5.45) (width 0.2) (layer "F.Cu") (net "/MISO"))
 (segment (start 6.5729 7.1021) (end 8.0242 7.1021) (width 0.2) (layer "F.Cu") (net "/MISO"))
 (segment (start 8.75 6.3763) (end 8.75 4.5236) (width 0.2) (layer "F.Cu") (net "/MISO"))
 (segment (start 5.175 8.5) (end 6.5729 7.1021) (width 0.2) (layer "F.Cu") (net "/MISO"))
 (segment (start 8.0242 7.1021) (end 8.75 6.3763) (width 0.2) (layer "F.Cu") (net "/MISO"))
 (segment (start 9.7609 4.2977) (end 10.625 5.1618) (width 0.2) (layer "F.Cu") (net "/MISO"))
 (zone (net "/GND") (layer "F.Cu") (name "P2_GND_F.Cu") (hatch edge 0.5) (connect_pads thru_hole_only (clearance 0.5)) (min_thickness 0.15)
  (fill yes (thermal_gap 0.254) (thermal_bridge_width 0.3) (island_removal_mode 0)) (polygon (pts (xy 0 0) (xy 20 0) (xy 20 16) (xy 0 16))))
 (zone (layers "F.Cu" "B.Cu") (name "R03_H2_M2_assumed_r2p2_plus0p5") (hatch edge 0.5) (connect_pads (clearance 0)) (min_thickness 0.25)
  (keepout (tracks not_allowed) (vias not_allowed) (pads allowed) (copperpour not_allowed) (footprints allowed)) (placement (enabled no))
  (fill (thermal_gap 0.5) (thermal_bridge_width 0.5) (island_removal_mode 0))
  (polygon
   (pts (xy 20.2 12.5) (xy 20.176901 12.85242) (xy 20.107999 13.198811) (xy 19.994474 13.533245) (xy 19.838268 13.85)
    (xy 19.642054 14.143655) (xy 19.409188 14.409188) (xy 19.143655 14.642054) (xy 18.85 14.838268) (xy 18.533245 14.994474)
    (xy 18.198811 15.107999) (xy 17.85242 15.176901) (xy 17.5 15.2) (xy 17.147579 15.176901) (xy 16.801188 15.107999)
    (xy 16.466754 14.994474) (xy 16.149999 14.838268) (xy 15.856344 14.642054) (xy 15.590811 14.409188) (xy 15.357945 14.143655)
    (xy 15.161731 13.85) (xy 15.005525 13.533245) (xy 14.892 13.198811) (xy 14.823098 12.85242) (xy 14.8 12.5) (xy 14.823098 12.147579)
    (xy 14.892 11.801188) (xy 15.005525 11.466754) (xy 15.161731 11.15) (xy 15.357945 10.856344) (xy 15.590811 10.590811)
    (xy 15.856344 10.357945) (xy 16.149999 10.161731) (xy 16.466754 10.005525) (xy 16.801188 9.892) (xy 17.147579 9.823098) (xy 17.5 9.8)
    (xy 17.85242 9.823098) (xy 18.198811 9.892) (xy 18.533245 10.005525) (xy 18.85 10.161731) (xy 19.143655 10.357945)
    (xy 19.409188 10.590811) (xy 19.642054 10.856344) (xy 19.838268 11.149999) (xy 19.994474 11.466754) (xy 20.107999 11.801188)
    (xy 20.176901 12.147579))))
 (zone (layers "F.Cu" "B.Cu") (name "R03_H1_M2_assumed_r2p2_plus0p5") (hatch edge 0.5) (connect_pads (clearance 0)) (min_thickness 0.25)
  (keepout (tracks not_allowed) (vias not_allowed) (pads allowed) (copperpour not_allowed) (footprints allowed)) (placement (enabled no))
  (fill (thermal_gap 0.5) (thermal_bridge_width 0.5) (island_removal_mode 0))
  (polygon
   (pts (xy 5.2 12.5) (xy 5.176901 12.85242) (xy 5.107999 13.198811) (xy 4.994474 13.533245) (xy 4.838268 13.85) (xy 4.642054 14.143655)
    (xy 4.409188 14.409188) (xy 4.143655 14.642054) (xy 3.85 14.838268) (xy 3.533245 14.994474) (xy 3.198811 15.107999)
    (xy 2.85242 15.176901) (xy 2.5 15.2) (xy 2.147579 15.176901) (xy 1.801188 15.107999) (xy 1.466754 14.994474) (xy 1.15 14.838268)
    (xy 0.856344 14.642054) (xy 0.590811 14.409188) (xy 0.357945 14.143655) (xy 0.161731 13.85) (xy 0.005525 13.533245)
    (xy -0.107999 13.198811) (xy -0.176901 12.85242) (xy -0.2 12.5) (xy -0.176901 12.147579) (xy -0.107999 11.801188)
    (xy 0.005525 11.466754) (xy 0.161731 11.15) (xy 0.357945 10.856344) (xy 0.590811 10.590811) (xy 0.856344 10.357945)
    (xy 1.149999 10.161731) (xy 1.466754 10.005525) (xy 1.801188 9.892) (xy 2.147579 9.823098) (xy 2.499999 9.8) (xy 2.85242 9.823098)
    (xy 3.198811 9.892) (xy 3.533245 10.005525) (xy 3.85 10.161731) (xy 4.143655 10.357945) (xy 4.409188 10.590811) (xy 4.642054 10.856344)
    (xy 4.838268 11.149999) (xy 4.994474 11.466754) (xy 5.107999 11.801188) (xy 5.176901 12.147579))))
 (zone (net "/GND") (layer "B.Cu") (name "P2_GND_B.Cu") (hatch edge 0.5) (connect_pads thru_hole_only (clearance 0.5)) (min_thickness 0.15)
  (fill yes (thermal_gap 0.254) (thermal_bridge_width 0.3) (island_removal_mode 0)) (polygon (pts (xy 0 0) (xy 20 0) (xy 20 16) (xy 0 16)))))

